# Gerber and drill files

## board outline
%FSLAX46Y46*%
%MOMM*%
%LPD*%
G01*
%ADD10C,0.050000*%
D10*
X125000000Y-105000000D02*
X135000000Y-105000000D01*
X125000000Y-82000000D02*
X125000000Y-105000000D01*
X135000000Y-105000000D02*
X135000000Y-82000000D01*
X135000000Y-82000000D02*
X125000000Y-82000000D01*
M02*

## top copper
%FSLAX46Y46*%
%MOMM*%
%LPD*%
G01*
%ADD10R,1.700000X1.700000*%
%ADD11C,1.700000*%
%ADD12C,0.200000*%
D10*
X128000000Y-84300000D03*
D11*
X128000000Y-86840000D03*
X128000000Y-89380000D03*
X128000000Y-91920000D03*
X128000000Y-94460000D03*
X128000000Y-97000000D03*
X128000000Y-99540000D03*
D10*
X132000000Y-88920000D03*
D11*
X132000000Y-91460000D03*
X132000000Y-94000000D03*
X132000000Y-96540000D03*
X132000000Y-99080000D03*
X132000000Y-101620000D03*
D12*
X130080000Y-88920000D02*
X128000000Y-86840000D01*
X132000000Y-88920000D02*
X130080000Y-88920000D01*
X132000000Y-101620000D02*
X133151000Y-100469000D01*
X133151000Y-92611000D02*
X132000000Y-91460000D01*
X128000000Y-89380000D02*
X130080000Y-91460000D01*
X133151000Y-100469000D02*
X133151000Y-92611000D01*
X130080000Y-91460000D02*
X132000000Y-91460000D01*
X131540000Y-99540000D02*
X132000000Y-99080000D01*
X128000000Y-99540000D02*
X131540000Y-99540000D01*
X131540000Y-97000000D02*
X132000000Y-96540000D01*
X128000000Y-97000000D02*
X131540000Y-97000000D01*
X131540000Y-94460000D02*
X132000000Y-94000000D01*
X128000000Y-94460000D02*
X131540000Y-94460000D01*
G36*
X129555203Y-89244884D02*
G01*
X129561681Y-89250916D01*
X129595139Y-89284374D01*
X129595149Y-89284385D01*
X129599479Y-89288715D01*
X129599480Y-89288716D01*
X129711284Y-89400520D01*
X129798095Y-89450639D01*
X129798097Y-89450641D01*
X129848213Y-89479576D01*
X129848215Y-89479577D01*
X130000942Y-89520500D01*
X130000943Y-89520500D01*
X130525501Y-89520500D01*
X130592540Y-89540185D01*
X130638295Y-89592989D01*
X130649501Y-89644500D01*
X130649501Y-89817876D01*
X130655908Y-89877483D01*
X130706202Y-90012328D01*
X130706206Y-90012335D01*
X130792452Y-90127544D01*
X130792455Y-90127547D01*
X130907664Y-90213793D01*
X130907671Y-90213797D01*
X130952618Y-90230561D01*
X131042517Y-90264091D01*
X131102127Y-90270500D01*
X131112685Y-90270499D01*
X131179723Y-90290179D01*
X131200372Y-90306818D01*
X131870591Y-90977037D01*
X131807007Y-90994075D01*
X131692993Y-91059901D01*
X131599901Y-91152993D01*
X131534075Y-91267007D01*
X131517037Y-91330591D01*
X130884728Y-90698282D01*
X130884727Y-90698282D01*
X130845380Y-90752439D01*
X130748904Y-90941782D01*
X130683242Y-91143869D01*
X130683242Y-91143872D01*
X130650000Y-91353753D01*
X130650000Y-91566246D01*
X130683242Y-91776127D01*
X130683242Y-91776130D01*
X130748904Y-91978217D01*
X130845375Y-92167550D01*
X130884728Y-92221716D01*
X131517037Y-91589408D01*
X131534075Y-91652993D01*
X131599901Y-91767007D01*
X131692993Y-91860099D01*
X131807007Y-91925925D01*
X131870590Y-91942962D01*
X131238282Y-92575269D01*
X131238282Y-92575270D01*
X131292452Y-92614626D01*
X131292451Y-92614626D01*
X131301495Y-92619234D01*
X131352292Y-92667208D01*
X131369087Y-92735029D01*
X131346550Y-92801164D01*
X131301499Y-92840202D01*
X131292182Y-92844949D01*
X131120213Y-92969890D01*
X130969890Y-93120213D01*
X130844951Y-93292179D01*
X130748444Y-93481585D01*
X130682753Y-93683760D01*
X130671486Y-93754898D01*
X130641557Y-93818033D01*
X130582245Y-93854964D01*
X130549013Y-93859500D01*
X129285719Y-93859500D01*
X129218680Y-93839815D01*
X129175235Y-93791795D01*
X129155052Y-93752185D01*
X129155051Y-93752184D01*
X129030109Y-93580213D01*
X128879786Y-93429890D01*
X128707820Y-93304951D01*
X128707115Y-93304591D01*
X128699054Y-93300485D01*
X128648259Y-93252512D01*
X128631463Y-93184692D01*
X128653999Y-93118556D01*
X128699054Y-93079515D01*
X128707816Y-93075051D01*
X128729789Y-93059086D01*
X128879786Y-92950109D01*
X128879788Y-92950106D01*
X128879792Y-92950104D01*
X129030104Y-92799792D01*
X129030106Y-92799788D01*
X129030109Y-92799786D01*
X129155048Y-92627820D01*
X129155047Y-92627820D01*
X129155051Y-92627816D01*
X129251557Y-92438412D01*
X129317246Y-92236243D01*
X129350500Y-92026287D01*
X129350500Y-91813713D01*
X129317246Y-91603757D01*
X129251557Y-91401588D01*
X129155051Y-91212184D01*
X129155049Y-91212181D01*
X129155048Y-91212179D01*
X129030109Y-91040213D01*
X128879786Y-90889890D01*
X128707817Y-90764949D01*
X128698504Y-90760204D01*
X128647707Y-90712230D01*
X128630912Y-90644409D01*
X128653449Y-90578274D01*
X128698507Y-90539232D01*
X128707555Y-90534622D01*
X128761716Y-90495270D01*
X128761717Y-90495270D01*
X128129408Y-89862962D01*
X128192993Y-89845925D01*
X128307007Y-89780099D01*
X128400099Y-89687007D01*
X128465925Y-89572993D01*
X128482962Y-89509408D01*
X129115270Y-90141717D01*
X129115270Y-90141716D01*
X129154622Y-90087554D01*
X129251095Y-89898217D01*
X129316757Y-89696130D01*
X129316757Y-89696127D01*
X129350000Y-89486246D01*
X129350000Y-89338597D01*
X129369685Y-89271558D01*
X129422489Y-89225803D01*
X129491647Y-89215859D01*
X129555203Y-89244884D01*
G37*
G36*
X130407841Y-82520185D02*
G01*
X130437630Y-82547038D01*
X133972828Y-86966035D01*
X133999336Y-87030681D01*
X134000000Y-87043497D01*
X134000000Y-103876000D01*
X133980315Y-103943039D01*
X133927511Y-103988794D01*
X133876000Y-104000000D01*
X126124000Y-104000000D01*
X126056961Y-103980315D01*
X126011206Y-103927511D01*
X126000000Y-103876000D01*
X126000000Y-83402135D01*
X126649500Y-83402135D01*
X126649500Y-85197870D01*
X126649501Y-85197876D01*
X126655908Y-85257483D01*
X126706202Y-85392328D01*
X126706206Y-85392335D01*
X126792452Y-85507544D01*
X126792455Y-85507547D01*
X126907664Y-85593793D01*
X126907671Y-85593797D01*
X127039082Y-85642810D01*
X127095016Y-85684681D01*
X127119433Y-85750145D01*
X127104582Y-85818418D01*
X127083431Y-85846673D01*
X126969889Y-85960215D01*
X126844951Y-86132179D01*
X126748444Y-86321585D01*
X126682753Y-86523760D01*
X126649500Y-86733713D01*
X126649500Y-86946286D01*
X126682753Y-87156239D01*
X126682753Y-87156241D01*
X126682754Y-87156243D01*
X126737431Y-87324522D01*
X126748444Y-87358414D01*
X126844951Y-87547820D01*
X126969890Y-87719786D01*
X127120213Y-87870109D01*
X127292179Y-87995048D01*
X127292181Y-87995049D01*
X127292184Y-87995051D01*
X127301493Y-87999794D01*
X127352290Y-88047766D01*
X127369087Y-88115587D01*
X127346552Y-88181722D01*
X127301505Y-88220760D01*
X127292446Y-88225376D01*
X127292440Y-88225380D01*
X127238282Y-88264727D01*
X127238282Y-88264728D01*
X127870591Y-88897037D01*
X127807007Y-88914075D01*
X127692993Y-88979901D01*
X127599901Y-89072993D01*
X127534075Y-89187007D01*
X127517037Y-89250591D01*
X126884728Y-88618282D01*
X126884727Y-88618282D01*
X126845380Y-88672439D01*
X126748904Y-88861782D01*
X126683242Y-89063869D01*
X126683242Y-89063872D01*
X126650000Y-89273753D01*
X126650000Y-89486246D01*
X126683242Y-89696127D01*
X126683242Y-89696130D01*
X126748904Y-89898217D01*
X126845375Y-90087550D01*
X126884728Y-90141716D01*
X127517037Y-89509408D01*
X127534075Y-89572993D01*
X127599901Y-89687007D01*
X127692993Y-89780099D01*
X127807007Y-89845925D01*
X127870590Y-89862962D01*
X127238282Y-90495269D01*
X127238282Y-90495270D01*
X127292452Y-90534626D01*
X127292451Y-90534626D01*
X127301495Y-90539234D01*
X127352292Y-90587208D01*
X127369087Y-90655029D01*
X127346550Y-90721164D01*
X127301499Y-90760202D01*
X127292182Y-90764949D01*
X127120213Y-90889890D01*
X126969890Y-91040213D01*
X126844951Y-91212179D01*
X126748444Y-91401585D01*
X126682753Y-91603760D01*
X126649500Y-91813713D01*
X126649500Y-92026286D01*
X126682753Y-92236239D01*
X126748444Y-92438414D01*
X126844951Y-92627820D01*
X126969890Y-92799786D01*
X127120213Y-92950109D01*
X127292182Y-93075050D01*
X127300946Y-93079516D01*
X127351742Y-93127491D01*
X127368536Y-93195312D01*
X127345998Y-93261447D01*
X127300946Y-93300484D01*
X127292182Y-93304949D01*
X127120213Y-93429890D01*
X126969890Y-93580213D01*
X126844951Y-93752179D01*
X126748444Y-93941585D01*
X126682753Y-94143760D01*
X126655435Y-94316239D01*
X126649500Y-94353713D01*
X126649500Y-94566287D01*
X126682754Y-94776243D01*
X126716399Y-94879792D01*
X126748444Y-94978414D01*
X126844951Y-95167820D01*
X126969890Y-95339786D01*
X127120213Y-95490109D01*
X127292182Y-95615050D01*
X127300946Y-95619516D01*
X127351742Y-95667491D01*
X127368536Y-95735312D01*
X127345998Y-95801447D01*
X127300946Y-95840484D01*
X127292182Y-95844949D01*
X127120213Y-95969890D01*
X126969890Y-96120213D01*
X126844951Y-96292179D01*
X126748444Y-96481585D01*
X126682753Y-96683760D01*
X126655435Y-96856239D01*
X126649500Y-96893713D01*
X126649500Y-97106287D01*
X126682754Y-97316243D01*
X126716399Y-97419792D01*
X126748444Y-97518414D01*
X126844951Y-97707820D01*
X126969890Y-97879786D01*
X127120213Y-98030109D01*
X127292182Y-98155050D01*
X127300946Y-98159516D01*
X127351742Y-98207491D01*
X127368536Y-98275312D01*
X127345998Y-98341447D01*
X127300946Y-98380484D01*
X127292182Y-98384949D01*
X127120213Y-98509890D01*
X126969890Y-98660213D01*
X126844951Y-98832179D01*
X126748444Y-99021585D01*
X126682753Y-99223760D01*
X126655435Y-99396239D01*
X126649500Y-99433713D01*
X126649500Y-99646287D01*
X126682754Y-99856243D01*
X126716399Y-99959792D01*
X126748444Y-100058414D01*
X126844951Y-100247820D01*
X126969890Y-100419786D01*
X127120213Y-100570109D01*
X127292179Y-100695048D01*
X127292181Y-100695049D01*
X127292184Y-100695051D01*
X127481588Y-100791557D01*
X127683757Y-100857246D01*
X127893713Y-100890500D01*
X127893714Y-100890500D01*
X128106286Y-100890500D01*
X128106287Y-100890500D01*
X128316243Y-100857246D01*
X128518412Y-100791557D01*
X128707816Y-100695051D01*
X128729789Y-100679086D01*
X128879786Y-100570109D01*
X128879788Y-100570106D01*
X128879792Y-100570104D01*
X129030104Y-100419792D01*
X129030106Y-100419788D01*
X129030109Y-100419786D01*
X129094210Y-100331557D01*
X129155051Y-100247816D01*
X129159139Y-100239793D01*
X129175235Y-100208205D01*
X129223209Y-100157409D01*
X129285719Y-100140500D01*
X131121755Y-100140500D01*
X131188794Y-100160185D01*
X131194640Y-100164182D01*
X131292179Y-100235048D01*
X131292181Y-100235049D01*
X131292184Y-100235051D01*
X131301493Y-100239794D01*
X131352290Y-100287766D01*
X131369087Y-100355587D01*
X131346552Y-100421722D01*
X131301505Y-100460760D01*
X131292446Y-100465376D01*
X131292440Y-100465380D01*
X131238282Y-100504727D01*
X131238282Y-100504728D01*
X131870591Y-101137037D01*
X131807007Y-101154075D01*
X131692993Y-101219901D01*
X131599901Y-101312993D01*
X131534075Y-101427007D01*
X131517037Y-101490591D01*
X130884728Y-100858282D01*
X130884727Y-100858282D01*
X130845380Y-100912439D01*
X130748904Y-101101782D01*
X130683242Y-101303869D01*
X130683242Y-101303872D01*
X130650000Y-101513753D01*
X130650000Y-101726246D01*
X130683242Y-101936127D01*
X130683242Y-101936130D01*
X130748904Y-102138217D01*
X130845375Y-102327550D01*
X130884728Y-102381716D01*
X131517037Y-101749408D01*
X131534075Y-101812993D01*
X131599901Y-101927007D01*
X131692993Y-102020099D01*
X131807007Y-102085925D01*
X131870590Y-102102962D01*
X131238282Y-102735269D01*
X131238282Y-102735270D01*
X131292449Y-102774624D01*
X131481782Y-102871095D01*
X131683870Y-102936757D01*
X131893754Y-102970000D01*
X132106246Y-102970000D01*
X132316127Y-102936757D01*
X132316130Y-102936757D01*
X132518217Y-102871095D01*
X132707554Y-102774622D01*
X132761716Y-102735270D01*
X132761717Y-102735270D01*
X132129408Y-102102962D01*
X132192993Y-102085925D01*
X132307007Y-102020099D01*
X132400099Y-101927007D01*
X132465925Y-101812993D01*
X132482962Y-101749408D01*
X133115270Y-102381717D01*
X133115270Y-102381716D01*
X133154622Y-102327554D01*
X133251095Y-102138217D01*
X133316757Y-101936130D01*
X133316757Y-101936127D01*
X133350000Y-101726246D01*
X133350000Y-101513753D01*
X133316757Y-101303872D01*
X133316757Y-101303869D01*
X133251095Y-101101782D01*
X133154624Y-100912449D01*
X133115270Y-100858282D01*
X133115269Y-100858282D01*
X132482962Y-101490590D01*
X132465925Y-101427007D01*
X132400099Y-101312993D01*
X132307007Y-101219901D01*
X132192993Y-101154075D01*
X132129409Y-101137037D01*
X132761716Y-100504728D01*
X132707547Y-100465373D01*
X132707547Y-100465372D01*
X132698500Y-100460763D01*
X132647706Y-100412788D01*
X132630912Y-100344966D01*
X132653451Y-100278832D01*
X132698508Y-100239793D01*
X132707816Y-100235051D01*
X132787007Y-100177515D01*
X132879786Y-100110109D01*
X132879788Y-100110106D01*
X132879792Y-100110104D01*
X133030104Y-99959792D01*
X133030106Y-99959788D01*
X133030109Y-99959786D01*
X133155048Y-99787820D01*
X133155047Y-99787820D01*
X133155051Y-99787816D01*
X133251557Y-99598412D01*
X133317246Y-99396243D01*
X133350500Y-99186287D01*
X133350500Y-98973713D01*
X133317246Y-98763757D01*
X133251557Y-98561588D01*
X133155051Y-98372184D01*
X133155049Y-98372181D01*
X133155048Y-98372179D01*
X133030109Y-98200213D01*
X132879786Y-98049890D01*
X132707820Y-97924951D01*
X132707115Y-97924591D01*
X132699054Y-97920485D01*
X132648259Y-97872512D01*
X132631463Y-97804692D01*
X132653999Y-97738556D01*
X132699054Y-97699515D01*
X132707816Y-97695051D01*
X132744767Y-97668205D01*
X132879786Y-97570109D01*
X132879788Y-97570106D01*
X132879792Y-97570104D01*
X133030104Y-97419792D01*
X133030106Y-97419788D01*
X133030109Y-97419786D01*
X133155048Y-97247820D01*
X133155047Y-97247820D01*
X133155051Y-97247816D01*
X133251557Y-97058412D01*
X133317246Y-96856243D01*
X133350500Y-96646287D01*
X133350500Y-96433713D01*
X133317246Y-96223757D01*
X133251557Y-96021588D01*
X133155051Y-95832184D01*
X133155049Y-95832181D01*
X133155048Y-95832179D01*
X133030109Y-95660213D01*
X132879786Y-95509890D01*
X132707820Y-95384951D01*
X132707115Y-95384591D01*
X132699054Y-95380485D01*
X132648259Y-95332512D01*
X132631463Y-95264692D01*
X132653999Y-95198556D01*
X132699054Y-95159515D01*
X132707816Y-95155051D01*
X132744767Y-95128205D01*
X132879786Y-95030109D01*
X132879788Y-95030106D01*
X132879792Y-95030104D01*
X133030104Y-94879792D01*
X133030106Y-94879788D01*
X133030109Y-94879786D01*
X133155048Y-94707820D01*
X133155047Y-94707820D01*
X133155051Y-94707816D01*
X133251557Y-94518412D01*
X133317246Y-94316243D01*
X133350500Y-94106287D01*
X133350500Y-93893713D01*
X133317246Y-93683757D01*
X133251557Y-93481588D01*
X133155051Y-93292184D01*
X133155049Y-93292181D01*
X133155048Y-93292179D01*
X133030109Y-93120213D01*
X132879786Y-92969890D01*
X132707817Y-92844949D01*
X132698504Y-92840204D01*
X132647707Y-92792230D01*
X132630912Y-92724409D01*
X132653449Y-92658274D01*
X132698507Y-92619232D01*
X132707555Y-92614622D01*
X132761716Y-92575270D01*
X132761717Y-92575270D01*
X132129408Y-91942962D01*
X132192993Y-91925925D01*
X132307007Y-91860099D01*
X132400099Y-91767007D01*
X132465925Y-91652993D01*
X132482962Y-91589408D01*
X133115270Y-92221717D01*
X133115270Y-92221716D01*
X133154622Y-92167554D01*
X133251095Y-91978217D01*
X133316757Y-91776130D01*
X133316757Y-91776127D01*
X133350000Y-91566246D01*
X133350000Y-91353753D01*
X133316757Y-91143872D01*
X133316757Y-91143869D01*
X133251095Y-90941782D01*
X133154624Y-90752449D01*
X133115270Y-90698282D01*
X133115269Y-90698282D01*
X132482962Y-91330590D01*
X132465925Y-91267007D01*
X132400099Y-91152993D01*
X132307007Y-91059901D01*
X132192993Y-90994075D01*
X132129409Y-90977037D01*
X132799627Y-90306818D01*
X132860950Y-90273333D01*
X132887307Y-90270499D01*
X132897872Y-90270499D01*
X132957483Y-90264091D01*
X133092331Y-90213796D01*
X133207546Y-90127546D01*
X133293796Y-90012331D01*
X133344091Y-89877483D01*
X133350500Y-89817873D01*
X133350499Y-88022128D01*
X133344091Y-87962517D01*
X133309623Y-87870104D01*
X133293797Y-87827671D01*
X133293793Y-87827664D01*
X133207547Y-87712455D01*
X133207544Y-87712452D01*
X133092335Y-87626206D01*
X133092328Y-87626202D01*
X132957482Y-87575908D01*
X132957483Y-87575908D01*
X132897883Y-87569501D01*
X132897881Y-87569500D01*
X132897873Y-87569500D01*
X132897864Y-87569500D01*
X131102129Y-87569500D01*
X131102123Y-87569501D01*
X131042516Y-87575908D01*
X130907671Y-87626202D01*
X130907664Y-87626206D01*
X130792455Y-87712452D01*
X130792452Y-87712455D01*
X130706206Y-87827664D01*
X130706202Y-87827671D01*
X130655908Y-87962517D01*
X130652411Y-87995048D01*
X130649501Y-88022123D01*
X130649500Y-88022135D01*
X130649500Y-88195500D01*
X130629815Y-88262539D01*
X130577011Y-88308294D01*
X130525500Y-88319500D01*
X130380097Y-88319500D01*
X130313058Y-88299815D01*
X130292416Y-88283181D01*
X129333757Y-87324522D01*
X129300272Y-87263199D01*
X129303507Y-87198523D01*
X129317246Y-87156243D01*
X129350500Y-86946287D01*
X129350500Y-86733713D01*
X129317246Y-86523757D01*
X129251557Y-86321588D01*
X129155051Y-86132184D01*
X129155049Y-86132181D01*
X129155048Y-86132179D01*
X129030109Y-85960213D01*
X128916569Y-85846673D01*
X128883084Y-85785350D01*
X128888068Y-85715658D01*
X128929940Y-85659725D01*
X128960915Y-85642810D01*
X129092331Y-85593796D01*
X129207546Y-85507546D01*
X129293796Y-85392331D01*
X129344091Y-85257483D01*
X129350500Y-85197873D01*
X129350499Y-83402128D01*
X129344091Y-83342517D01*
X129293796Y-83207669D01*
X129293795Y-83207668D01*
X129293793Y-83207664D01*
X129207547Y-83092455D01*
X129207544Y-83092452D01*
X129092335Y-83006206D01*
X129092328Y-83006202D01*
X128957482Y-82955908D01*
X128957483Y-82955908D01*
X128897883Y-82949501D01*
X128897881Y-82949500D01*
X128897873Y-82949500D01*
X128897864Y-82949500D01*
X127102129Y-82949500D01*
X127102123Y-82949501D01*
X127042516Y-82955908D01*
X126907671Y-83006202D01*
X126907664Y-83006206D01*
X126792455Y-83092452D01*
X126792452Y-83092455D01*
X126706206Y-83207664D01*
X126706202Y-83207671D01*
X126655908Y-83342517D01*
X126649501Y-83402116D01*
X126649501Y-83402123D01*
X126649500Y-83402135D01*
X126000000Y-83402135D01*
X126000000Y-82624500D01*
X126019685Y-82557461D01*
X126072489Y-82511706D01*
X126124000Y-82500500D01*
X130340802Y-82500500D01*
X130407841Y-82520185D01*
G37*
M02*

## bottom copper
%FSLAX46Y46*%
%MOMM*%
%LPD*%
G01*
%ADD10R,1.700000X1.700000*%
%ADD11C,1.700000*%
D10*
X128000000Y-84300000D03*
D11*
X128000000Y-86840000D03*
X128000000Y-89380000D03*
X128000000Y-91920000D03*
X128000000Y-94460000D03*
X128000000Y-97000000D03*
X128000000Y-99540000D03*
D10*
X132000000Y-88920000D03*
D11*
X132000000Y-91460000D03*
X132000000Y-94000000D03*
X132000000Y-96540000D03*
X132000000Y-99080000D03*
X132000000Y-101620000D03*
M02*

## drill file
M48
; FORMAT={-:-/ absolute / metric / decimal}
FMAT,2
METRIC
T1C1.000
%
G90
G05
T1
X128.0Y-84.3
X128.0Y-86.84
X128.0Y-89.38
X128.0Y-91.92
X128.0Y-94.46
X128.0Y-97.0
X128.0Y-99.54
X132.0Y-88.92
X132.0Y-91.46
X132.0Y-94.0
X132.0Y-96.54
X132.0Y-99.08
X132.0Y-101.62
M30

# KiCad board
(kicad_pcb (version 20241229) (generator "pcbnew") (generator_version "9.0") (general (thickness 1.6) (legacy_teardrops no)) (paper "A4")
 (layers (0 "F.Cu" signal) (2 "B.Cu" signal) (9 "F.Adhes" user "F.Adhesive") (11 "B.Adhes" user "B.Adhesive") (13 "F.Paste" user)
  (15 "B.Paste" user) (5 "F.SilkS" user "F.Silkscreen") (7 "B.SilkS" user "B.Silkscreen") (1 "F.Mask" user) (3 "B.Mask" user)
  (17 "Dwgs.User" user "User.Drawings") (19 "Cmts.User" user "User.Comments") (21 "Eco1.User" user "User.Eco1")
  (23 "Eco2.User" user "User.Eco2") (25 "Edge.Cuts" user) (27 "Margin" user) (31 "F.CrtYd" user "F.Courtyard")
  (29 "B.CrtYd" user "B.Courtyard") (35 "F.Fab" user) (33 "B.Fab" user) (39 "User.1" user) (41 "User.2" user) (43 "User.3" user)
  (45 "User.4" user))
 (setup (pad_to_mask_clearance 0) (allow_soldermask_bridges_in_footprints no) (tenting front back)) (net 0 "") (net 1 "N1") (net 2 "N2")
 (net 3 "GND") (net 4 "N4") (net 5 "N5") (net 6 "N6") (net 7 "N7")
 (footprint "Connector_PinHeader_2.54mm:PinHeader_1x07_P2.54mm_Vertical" (layer "F.Cu") (at 128 84.3)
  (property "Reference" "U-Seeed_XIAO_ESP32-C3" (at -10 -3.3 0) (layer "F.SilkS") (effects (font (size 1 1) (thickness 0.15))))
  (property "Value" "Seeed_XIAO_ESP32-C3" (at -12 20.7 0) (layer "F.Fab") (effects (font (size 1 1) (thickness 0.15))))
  (pad "1" thru_hole rect (at 0 0) (size 1.7 1.7) (drill 1) (layers "*.Cu" "*.Mask") (remove_unused_layers no) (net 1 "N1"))
  (pad "2" thru_hole circle (at 0 2.54) (size 1.7 1.7) (drill 1) (layers "*.Cu" "*.Mask") (remove_unused_layers no) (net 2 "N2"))
  (pad "3" thru_hole circle (at 0 5.08) (size 1.7 1.7) (drill 1) (layers "*.Cu" "*.Mask") (remove_unused_layers no) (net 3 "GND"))
  (pad "4" thru_hole circle (at 0 7.62) (size 1.7 1.7) (drill 1) (layers "*.Cu" "*.Mask") (remove_unused_layers no) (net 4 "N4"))
  (pad "5" thru_hole circle (at 0 10.16) (size 1.7 1.7) (drill 1) (layers "*.Cu" "*.Mask") (remove_unused_layers no) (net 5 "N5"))
  (pad "6" thru_hole circle (at 0 12.7) (size 1.7 1.7) (drill 1) (layers "*.Cu" "*.Mask") (remove_unused_layers no) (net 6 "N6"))
  (pad "7" thru_hole circle (at 0 15.24) (size 1.7 1.7) (drill 1) (layers "*.Cu" "*.Mask") (remove_unused_layers no) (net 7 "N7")))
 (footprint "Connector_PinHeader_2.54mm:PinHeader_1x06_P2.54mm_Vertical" (layer "F.Cu") (at 132 88.92)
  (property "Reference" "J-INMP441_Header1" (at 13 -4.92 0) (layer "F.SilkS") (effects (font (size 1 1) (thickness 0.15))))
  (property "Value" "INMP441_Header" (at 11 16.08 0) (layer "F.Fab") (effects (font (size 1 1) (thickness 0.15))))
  (pad "1" thru_hole rect (at 0 0) (size 1.7 1.7) (drill 1) (layers "*.Cu" "*.Mask") (remove_unused_layers no) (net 2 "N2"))
  (pad "2" thru_hole circle (at 0 2.54) (size 1.7 1.7) (drill 1) (layers "*.Cu" "*.Mask") (remove_unused_layers no) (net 3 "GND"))
  (pad "3" thru_hole circle (at 0 5.08) (size 1.7 1.7) (drill 1) (layers "*.Cu" "*.Mask") (remove_unused_layers no) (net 5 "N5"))
  (pad "4" thru_hole circle (at 0 7.62) (size 1.7 1.7) (drill 1) (layers "*.Cu" "*.Mask") (remove_unused_layers no) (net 6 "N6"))
  (pad "5" thru_hole circle (at 0 10.16) (size 1.7 1.7) (drill 1) (layers "*.Cu" "*.Mask") (remove_unused_layers no) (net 7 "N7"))
  (pad "6" thru_hole circle (at 0 12.7) (size 1.7 1.7) (drill 1) (layers "*.Cu" "*.Mask") (remove_unused_layers no) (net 3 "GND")))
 (gr_line (start 125 105) (end 135 105) (stroke (width 0.05) (type default)) (layer "Edge.Cuts"))
 (gr_line (start 125 82) (end 125 105) (stroke (width 0.05) (type default)) (layer "Edge.Cuts"))
 (gr_line (start 135 105) (end 135 82) (stroke (width 0.05) (type default)) (layer "Edge.Cuts"))
 (gr_line (start 135 82) (end 125 82) (stroke (width 0.05) (type default)) (layer "Edge.Cuts"))
 (segment (start 130.08 88.92) (end 128 86.84) (width 0.2) (layer "F.Cu") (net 2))
 (segment (start 132 88.92) (end 130.08 88.92) (width 0.2) (layer "F.Cu") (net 2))
 (segment (start 132 101.62) (end 133.151 100.469) (width 0.2) (layer "F.Cu") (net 3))
 (segment (start 133.151 92.611) (end 132 91.46) (width 0.2) (layer "F.Cu") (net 3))
 (segment (start 128 89.38) (end 130.08 91.46) (width 0.2) (layer "F.Cu") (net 3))
 (segment (start 133.151 100.469) (end 133.151 92.611) (width 0.2) (layer "F.Cu") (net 3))
 (segment (start 130.08 91.46) (end 132 91.46) (width 0.2) (layer "F.Cu") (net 3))
 (segment (start 131.54 99.54) (end 132 99.08) (width 0.2) (layer "F.Cu") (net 7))
 (segment (start 128 99.54) (end 131.54 99.54) (width 0.2) (layer "F.Cu") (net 7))
 (segment (start 131.54 97) (end 132 96.54) (width 0.2) (layer "F.Cu") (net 6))
 (segment (start 128 97) (end 131.54 97) (width 0.2) (layer "F.Cu") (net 6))
 (segment (start 131.54 94.46) (end 132 94) (width 0.2) (layer "F.Cu") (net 5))
 (segment (start 128 94.46) (end 131.54 94.46) (width 0.2) (layer "F.Cu") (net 5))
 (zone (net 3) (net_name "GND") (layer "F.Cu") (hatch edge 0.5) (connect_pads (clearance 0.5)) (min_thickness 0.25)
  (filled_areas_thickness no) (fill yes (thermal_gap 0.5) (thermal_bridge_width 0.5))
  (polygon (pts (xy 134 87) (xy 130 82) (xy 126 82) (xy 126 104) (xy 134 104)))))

